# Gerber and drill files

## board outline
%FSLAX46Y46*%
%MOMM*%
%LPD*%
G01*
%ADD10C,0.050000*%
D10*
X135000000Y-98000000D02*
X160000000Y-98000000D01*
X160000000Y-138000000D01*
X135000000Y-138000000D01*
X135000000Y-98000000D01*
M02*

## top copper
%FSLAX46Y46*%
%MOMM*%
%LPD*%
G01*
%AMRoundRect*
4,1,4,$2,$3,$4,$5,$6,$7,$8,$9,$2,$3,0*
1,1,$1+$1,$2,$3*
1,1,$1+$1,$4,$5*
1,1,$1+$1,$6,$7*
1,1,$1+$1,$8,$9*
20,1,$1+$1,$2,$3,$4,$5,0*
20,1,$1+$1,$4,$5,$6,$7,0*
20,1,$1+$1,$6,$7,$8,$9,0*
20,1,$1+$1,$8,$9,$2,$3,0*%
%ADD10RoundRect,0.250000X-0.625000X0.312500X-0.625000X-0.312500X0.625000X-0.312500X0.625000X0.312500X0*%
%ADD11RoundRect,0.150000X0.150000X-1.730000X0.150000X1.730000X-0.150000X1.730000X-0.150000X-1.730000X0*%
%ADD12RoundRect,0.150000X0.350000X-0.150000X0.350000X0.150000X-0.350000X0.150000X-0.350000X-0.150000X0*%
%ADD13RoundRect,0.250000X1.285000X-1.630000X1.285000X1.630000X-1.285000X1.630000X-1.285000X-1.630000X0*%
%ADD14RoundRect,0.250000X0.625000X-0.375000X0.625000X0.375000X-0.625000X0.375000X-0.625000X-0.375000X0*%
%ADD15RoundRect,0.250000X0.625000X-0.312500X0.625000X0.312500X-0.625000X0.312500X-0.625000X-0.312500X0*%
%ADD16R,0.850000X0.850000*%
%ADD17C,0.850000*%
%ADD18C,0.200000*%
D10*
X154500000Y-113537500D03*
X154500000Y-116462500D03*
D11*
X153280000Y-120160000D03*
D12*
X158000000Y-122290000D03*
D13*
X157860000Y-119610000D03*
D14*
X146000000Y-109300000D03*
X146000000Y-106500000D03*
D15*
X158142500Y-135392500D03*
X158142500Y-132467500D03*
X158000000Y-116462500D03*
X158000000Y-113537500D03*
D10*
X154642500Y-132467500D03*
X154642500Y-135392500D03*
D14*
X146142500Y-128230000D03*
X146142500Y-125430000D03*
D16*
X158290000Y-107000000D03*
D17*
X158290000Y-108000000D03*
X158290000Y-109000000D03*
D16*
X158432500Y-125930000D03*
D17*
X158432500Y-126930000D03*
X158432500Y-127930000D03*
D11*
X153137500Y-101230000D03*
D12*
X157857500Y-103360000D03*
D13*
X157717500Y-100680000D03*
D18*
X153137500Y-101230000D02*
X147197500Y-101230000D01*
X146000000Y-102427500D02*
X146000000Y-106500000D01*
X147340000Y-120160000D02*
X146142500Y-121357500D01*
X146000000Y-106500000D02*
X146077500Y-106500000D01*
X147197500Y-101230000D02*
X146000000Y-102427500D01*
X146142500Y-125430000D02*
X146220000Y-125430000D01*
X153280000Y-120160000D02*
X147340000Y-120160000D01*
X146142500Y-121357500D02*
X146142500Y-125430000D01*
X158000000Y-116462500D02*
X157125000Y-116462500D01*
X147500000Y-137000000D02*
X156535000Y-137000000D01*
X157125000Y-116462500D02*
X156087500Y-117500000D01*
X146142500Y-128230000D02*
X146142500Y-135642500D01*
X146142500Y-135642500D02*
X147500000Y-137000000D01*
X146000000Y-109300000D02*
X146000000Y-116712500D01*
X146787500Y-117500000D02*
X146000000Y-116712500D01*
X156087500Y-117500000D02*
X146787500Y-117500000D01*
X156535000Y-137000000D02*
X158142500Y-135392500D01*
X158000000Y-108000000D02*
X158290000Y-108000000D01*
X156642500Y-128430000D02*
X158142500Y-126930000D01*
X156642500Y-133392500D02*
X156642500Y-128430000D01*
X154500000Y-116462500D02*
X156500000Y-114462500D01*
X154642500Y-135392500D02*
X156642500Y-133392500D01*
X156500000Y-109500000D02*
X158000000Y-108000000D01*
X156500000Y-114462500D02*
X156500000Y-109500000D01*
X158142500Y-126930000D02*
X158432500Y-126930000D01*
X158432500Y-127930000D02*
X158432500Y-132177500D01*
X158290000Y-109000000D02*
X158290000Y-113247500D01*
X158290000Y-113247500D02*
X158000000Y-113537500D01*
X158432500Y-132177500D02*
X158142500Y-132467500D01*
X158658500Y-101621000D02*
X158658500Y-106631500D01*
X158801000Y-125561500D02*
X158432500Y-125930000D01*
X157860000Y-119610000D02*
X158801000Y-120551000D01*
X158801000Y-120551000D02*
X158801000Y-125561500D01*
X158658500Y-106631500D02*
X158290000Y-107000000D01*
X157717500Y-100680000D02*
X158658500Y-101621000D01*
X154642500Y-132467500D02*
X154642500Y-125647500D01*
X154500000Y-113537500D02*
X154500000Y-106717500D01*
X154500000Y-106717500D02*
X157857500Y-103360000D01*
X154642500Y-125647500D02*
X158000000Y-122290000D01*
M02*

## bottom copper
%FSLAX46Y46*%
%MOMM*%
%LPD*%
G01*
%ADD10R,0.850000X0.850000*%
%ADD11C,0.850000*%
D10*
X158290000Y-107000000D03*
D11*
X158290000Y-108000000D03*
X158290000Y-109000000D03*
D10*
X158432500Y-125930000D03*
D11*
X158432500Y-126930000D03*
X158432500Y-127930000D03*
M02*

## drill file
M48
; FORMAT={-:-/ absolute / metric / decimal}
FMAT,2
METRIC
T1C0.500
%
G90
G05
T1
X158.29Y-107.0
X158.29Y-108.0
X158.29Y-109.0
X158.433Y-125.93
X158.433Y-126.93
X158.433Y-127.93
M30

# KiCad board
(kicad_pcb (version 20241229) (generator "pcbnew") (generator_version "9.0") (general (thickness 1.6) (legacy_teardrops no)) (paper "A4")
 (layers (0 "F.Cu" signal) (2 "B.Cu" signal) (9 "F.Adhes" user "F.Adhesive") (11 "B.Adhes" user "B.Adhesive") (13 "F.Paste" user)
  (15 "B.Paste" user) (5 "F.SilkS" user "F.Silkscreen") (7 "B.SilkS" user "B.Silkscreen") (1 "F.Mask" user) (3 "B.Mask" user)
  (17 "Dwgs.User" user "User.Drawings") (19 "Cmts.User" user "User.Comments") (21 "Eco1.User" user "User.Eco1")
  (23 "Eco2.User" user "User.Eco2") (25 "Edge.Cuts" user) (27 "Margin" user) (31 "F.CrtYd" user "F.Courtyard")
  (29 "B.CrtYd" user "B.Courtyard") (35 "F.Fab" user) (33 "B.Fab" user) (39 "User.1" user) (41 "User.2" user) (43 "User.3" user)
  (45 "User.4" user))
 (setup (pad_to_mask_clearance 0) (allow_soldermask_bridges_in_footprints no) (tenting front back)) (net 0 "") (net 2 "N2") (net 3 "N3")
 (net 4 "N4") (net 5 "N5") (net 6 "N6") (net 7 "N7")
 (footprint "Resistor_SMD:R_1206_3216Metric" (layer "F.Cu") (at 154.5 115 -90)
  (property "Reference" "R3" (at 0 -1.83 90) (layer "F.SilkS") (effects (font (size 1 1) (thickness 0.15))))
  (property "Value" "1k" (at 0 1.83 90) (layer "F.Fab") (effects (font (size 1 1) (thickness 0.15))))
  (pad "1" smd roundrect (at -1.4625 0 270) (size 1.125 1.75) (layers "F.Cu" "F.Mask" "F.Paste") (roundrect_rratio 0.222222) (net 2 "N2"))
  (pad "2" smd roundrect (at 1.4625 0 270) (size 1.125 1.75) (layers "F.Cu" "F.Mask" "F.Paste") (roundrect_rratio 0.222222) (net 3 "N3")))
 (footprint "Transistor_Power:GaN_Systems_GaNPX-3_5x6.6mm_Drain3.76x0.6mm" (layer "F.Cu") (at 156.19 120.16 90)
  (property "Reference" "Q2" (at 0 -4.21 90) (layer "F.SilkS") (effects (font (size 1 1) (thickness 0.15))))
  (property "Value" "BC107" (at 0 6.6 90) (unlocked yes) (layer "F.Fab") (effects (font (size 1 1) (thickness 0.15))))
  (pad "" smd roundrect (at -0.34 0.9525 90) (size 1.58 1.235) (layers "F.Paste") (roundrect_rratio 0.2024291498))
  (pad "" smd roundrect (at -0.34 2.3875 90) (size 1.58 1.235) (layers "F.Paste") (roundrect_rratio 0.2024291498))
  (pad "" smd roundrect (at 1.44 0.9525 90) (size 1.58 1.235) (layers "F.Paste") (roundrect_rratio 0.2024291498))
  (pad "" smd roundrect (at 1.44 2.3875 90) (size 1.58 1.235) (layers "F.Paste") (roundrect_rratio 0.2024291498))
  (pad "1" smd roundrect (at 0 -2.91 90) (size 3.76 0.6) (layers "F.Cu" "F.Mask" "F.Paste") (roundrect_rratio 0.25) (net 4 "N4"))
  (pad "2" smd roundrect (at -2.13 1.81 90) (size 0.6 1) (layers "F.Cu" "F.Mask" "F.Paste") (roundrect_rratio 0.25) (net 2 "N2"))
  (pad "3" smd roundrect (at 0.55 1.67 90) (size 3.76 3.07) (layers "F.Cu" "F.Mask") (roundrect_rratio 0.08143322476) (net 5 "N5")))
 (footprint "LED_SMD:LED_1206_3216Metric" (layer "F.Cu") (at 146 107.9 90)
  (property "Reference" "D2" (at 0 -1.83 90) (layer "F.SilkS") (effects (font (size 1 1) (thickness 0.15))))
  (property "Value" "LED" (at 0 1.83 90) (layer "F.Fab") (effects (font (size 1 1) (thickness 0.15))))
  (pad "1" smd roundrect (at -1.4 0 90) (size 1.25 1.75) (layers "F.Cu" "F.Mask" "F.Paste") (roundrect_rratio 0.2) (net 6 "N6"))
  (pad "2" smd roundrect (at 1.4 0 90) (size 1.25 1.75) (layers "F.Cu" "F.Mask" "F.Paste") (roundrect_rratio 0.2) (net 4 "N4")))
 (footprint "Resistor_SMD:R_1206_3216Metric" (layer "F.Cu") (at 158.1425 133.93 90)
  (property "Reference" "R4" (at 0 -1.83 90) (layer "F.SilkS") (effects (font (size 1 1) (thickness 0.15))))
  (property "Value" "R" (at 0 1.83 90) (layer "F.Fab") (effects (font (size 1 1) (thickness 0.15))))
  (pad "1" smd roundrect (at -1.4625 0 90) (size 1.125 1.75) (layers "F.Cu" "F.Mask" "F.Paste") (roundrect_rratio 0.222222) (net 6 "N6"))
  (pad "2" smd roundrect (at 1.4625 0 90) (size 1.125 1.75) (layers "F.Cu" "F.Mask" "F.Paste") (roundrect_rratio 0.222222) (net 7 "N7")))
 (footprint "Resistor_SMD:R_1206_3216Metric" (layer "F.Cu") (at 158 115 90)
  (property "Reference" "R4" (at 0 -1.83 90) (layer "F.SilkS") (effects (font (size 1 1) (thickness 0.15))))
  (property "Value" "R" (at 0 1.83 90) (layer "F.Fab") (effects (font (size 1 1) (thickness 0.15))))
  (pad "1" smd roundrect (at -1.4625 0 90) (size 1.125 1.75) (layers "F.Cu" "F.Mask" "F.Paste") (roundrect_rratio 0.222222) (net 6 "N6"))
  (pad "2" smd roundrect (at 1.4625 0 90) (size 1.125 1.75) (layers "F.Cu" "F.Mask" "F.Paste") (roundrect_rratio 0.222222) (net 7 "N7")))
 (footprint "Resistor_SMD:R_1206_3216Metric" (layer "F.Cu") (at 154.6425 133.93 -90)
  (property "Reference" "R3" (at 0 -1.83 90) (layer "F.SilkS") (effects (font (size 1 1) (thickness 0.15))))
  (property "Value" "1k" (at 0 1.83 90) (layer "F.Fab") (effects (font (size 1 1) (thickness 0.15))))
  (pad "1" smd roundrect (at -1.4625 0 270) (size 1.125 1.75) (layers "F.Cu" "F.Mask" "F.Paste") (roundrect_rratio 0.222222) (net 2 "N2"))
  (pad "2" smd roundrect (at 1.4625 0 270) (size 1.125 1.75) (layers "F.Cu" "F.Mask" "F.Paste") (roundrect_rratio 0.222222) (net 3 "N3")))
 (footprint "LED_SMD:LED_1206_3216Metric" (layer "F.Cu") (at 146.1425 126.83 90)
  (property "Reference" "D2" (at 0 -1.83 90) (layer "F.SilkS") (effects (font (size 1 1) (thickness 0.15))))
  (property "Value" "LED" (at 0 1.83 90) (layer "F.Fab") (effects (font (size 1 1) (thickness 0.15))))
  (pad "1" smd roundrect (at -1.4 0 90) (size 1.25 1.75) (layers "F.Cu" "F.Mask" "F.Paste") (roundrect_rratio 0.2) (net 6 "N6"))
  (pad "2" smd roundrect (at 1.4 0 90) (size 1.25 1.75) (layers "F.Cu" "F.Mask" "F.Paste") (roundrect_rratio 0.2) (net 4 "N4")))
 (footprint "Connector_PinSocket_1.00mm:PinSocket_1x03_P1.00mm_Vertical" (layer "F.Cu") (at 158.29 107)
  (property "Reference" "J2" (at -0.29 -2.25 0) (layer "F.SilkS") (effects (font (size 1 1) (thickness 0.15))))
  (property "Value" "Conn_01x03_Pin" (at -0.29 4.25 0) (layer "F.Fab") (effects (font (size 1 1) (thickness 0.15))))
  (pad "1" thru_hole rect (at 0 0) (size 0.85 0.85) (drill 0.5) (layers "*.Cu" "*.Mask") (remove_unused_layers no) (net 5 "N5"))
  (pad "2" thru_hole circle (at 0 1) (size 0.85 0.85) (drill 0.5) (layers "*.Cu" "*.Mask") (remove_unused_layers no) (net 3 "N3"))
  (pad "3" thru_hole circle (at 0 2) (size 0.85 0.85) (drill 0.5) (layers "*.Cu" "*.Mask") (remove_unused_layers no) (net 7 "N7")))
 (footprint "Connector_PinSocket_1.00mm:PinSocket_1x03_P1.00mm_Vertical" (layer "F.Cu") (at 158.4325 125.93)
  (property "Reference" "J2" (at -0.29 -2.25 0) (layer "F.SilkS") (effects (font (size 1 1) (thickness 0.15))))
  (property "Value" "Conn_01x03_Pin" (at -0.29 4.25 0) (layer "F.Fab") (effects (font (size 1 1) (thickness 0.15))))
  (pad "1" thru_hole rect (at 0 0) (size 0.85 0.85) (drill 0.5) (layers "*.Cu" "*.Mask") (remove_unused_layers no) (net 5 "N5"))
  (pad "2" thru_hole circle (at 0 1) (size 0.85 0.85) (drill 0.5) (layers "*.Cu" "*.Mask") (remove_unused_layers no) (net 3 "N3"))
  (pad "3" thru_hole circle (at 0 2) (size 0.85 0.85) (drill 0.5) (layers "*.Cu" "*.Mask") (remove_unused_layers no) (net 7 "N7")))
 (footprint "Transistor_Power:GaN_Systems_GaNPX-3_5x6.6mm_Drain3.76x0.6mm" (layer "F.Cu") (at 156.0475 101.23 90)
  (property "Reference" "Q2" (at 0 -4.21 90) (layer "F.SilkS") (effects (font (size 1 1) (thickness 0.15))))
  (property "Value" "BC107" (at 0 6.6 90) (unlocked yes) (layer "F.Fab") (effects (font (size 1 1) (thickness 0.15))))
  (pad "" smd roundrect (at -0.34 0.9525 90) (size 1.58 1.235) (layers "F.Paste") (roundrect_rratio 0.2024291498))
  (pad "" smd roundrect (at -0.34 2.3875 90) (size 1.58 1.235) (layers "F.Paste") (roundrect_rratio 0.2024291498))
  (pad "" smd roundrect (at 1.44 0.9525 90) (size 1.58 1.235) (layers "F.Paste") (roundrect_rratio 0.2024291498))
  (pad "" smd roundrect (at 1.44 2.3875 90) (size 1.58 1.235) (layers "F.Paste") (roundrect_rratio 0.2024291498))
  (pad "1" smd roundrect (at 0 -2.91 90) (size 3.76 0.6) (layers "F.Cu" "F.Mask" "F.Paste") (roundrect_rratio 0.25) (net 4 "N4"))
  (pad "2" smd roundrect (at -2.13 1.81 90) (size 0.6 1) (layers "F.Cu" "F.Mask" "F.Paste") (roundrect_rratio 0.25) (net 2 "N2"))
  (pad "3" smd roundrect (at 0.55 1.67 90) (size 3.76 3.07) (layers "F.Cu" "F.Mask") (roundrect_rratio 0.08143322476) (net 5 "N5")))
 (gr_rect (start 135 98) (end 160 138) (stroke (width 0.05) (type solid)) (fill no) (layer "Edge.Cuts"))
 (segment (start 153.1375 101.23) (end 147.1975 101.23) (width 0.2) (layer "F.Cu") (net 4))
 (segment (start 146 102.4275) (end 146 106.5) (width 0.2) (layer "F.Cu") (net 4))
 (segment (start 147.34 120.16) (end 146.1425 121.3575) (width 0.2) (layer "F.Cu") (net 4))
 (segment (start 146 106.5) (end 146.0775 106.5) (width 0.2) (layer "F.Cu") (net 4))
 (segment (start 147.1975 101.23) (end 146 102.4275) (width 0.2) (layer "F.Cu") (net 4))
 (segment (start 146.1425 125.43) (end 146.22 125.43) (width 0.2) (layer "F.Cu") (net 4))
 (segment (start 153.28 120.16) (end 147.34 120.16) (width 0.2) (layer "F.Cu") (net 4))
 (segment (start 146.1425 121.3575) (end 146.1425 125.43) (width 0.2) (layer "F.Cu") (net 4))
 (segment (start 158 116.4625) (end 157.125 116.4625) (width 0.2) (layer "F.Cu") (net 6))
 (segment (start 147.5 137) (end 156.535 137) (width 0.2) (layer "F.Cu") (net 6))
 (segment (start 157.125 116.4625) (end 156.0875 117.5) (width 0.2) (layer "F.Cu") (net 6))
 (segment (start 146.1425 128.23) (end 146.1425 135.6425) (width 0.2) (layer "F.Cu") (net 6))
 (segment (start 146.1425 135.6425) (end 147.5 137) (width 0.2) (layer "F.Cu") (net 6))
 (segment (start 146 109.3) (end 146 116.7125) (width 0.2) (layer "F.Cu") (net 6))
 (segment (start 146.7875 117.5) (end 146 116.7125) (width 0.2) (layer "F.Cu") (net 6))
 (segment (start 156.0875 117.5) (end 146.7875 117.5) (width 0.2) (layer "F.Cu") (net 6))
 (segment (start 156.535 137) (end 158.1425 135.3925) (width 0.2) (layer "F.Cu") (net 6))
 (segment (start 158 108) (end 158.29 108) (width 0.2) (layer "F.Cu") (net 3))
 (segment (start 156.6425 128.43) (end 158.1425 126.93) (width 0.2) (layer "F.Cu") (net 3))
 (segment (start 156.6425 133.3925) (end 156.6425 128.43) (width 0.2) (layer "F.Cu") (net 3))
 (segment (start 154.5 116.4625) (end 156.5 114.4625) (width 0.2) (layer "F.Cu") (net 3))
 (segment (start 154.6425 135.3925) (end 156.6425 133.3925) (width 0.2) (layer "F.Cu") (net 3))
 (segment (start 156.5 109.5) (end 158 108) (width 0.2) (layer "F.Cu") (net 3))
 (segment (start 156.5 114.4625) (end 156.5 109.5) (width 0.2) (layer "F.Cu") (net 3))
 (segment (start 158.1425 126.93) (end 158.4325 126.93) (width 0.2) (layer "F.Cu") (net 3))
 (segment (start 158.4325 127.93) (end 158.4325 132.1775) (width 0.2) (layer "F.Cu") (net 7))
 (segment (start 158.29 109) (end 158.29 113.2475) (width 0.2) (layer "F.Cu") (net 7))
 (segment (start 158.29 113.2475) (end 158 113.5375) (width 0.2) (layer "F.Cu") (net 7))
 (segment (start 158.4325 132.1775) (end 158.1425 132.4675) (width 0.2) (layer "F.Cu") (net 7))
 (segment (start 158.6585 101.621) (end 158.6585 106.6315) (width 0.2) (layer "F.Cu") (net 5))
 (segment (start 158.801 125.5615) (end 158.4325 125.93) (width 0.2) (layer "F.Cu") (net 5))
 (segment (start 157.86 119.61) (end 158.801 120.551) (width 0.2) (layer "F.Cu") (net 5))
 (segment (start 158.801 120.551) (end 158.801 125.5615) (width 0.2) (layer "F.Cu") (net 5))
 (segment (start 158.6585 106.6315) (end 158.29 107) (width 0.2) (layer "F.Cu") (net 5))
 (segment (start 157.7175 100.68) (end 158.6585 101.621) (width 0.2) (layer "F.Cu") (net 5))
 (segment (start 154.6425 132.4675) (end 154.6425 125.6475) (width 0.2) (layer "F.Cu") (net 2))
 (segment (start 154.5 113.5375) (end 154.5 106.7175) (width 0.2) (layer "F.Cu") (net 2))
 (segment (start 154.5 106.7175) (end 157.8575 103.36) (width 0.2) (layer "F.Cu") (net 2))
 (segment (start 154.6425 125.6475) (end 158 122.29) (width 0.2) (layer "F.Cu") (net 2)))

